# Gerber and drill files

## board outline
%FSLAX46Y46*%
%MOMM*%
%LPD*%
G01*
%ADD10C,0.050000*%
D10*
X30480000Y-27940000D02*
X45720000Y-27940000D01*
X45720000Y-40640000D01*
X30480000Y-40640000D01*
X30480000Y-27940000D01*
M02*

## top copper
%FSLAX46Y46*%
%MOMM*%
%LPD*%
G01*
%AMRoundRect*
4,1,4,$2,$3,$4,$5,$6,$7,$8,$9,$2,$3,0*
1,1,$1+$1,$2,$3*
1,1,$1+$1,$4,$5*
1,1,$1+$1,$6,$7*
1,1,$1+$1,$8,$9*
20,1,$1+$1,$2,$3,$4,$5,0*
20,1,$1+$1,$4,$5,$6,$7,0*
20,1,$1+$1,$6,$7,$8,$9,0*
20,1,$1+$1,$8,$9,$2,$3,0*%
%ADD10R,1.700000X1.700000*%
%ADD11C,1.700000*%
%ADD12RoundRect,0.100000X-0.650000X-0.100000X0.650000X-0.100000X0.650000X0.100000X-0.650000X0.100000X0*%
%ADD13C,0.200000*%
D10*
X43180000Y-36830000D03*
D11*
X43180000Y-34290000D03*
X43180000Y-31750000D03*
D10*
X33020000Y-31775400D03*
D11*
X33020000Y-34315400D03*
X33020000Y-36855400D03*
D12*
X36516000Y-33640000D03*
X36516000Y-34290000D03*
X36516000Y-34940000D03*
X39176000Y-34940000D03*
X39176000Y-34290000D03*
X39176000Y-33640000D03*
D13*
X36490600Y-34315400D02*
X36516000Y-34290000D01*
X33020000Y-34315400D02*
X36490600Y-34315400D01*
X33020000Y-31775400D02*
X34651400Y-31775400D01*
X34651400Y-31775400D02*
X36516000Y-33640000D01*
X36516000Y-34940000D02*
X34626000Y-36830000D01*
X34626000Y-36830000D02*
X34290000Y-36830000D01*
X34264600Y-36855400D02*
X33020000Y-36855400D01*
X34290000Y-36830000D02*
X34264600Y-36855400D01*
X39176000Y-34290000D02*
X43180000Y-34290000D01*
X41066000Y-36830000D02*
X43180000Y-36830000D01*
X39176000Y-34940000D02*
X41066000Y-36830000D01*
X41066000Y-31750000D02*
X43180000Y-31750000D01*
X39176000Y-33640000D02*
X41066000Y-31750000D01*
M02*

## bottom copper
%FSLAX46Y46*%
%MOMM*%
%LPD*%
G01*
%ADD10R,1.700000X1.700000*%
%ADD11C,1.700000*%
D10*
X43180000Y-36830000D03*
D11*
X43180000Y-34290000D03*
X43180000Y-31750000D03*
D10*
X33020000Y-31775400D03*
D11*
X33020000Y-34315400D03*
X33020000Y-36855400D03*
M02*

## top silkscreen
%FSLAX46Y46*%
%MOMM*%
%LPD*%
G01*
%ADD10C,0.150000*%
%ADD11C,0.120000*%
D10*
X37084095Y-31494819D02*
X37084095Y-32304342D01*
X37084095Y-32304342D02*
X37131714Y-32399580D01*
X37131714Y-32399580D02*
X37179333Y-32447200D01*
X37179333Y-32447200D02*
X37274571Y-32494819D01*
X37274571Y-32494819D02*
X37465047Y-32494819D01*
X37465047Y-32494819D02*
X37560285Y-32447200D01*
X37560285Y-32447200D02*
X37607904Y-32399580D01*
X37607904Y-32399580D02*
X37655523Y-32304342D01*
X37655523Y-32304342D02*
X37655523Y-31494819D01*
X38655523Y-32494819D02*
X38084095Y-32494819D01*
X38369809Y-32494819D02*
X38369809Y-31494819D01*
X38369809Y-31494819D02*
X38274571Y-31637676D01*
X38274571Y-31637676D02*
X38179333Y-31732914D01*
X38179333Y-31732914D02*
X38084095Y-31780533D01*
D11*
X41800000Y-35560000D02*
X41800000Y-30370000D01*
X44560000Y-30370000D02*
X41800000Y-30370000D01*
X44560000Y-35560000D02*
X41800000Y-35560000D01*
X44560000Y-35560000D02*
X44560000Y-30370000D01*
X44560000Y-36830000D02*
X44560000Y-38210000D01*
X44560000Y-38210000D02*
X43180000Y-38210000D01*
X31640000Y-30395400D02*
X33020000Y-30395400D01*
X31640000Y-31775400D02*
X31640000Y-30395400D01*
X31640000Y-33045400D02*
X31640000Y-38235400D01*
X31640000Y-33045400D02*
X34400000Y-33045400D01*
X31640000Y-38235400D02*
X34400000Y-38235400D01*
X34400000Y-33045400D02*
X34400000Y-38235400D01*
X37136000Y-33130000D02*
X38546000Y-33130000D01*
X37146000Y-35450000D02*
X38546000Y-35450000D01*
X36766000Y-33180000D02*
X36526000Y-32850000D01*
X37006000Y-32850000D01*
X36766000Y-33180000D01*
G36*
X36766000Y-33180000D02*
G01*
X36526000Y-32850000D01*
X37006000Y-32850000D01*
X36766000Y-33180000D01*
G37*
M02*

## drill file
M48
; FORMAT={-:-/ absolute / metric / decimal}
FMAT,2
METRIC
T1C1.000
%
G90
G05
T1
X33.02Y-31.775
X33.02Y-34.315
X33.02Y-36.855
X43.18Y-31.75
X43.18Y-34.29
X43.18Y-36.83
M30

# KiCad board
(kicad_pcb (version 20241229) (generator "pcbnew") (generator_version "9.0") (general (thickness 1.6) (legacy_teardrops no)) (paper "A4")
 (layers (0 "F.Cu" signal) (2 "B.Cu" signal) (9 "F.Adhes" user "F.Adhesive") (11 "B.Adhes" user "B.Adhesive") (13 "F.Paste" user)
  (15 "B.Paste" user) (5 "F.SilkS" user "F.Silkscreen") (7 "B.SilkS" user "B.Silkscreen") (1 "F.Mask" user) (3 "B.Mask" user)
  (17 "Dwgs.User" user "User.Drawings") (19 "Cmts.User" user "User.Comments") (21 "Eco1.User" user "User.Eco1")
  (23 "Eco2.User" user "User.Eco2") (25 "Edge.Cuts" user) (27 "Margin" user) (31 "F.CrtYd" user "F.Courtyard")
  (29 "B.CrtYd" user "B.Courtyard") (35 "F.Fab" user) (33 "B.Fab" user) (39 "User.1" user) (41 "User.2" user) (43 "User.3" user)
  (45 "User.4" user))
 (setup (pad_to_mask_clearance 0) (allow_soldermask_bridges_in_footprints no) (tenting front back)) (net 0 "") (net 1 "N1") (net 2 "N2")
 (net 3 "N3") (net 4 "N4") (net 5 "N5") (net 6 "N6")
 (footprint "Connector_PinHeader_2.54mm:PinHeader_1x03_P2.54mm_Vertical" (layer "F.Cu") (at 43.18 36.83 180)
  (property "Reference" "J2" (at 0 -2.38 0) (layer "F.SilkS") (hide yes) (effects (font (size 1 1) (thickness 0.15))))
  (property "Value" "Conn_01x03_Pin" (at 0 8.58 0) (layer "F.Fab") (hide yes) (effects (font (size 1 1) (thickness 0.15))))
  (fp_line (start 1.38 1.27) (end 1.38 6.46) (stroke (width 0.12) (type solid)) (layer "F.SilkS"))
  (fp_line (start -1.38 6.46) (end 1.38 6.46) (stroke (width 0.12) (type solid)) (layer "F.SilkS"))
  (fp_line (start -1.38 1.27) (end 1.38 1.27) (stroke (width 0.12) (type solid)) (layer "F.SilkS"))
  (fp_line (start -1.38 1.27) (end -1.38 6.46) (stroke (width 0.12) (type solid)) (layer "F.SilkS"))
  (fp_line (start -1.38 0) (end -1.38 -1.38) (stroke (width 0.12) (type solid)) (layer "F.SilkS"))
  (fp_line (start -1.38 -1.38) (end 0 -1.38) (stroke (width 0.12) (type solid)) (layer "F.SilkS"))
  (pad "1" thru_hole rect (at 0 0 180) (size 1.7 1.7) (drill 1) (layers "*.Cu" "*.Mask") (remove_unused_layers no) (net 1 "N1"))
  (pad "2" thru_hole circle (at 0 2.54 180) (size 1.7 1.7) (drill 1) (layers "*.Cu" "*.Mask") (remove_unused_layers no) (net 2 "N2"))
  (pad "3" thru_hole circle (at 0 5.08 180) (size 1.7 1.7) (drill 1) (layers "*.Cu" "*.Mask") (remove_unused_layers no) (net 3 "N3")))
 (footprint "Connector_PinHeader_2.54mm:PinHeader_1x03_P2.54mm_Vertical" (layer "F.Cu") (at 33.02 31.7754)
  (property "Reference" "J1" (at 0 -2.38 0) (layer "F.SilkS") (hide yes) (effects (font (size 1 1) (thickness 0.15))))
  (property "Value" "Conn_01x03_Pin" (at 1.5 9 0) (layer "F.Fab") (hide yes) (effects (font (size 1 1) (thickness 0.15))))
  (fp_line (start -1.38 -1.38) (end 0 -1.38) (stroke (width 0.12) (type solid)) (layer "F.SilkS"))
  (fp_line (start -1.38 0) (end -1.38 -1.38) (stroke (width 0.12) (type solid)) (layer "F.SilkS"))
  (fp_line (start -1.38 1.27) (end -1.38 6.46) (stroke (width 0.12) (type solid)) (layer "F.SilkS"))
  (fp_line (start -1.38 1.27) (end 1.38 1.27) (stroke (width 0.12) (type solid)) (layer "F.SilkS"))
  (fp_line (start -1.38 6.46) (end 1.38 6.46) (stroke (width 0.12) (type solid)) (layer "F.SilkS"))
  (fp_line (start 1.38 1.27) (end 1.38 6.46) (stroke (width 0.12) (type solid)) (layer "F.SilkS"))
  (pad "1" thru_hole rect (at 0 0) (size 1.7 1.7) (drill 1) (layers "*.Cu" "*.Mask") (remove_unused_layers no) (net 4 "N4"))
  (pad "2" thru_hole circle (at 0 2.54) (size 1.7 1.7) (drill 1) (layers "*.Cu" "*.Mask") (remove_unused_layers no) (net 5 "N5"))
  (pad "3" thru_hole circle (at 0 5.08) (size 1.7 1.7) (drill 1) (layers "*.Cu" "*.Mask") (remove_unused_layers no) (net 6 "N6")))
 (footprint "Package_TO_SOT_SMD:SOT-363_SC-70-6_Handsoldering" (layer "F.Cu") (at 37.846 34.29)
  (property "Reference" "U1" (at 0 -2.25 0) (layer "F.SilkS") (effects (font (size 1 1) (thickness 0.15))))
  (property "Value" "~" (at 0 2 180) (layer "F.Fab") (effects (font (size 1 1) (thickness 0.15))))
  (fp_line (start -0.71 -1.16) (end 0.7 -1.16) (stroke (width 0.12) (type solid)) (layer "F.SilkS"))
  (fp_line (start -0.7 1.16) (end 0.7 1.16) (stroke (width 0.12) (type solid)) (layer "F.SilkS"))
  (fp_poly
   (pts (xy -1.08 -1.11) (xy -1.32 -1.44) (xy -0.84 -1.44) (xy -1.08 -1.11)) (stroke (width 0.12) (type solid)) (fill yes) (layer "F.SilkS"))
  (pad "1" smd roundrect (at -1.33 -0.65) (size 1.5 0.4) (layers "F.Cu" "F.Mask" "F.Paste") (roundrect_rratio 0.25) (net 4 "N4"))
  (pad "2" smd roundrect (at -1.33 0) (size 1.5 0.4) (layers "F.Cu" "F.Mask" "F.Paste") (roundrect_rratio 0.25) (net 5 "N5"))
  (pad "3" smd roundrect (at -1.33 0.65) (size 1.5 0.4) (layers "F.Cu" "F.Mask" "F.Paste") (roundrect_rratio 0.25) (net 6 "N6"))
  (pad "4" smd roundrect (at 1.33 0.65) (size 1.5 0.4) (layers "F.Cu" "F.Mask" "F.Paste") (roundrect_rratio 0.25) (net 1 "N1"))
  (pad "5" smd roundrect (at 1.33 0) (size 1.5 0.4) (layers "F.Cu" "F.Mask" "F.Paste") (roundrect_rratio 0.25) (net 2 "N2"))
  (pad "6" smd roundrect (at 1.33 -0.65) (size 1.5 0.4) (layers "F.Cu" "F.Mask" "F.Paste") (roundrect_rratio 0.25) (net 3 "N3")))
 (gr_rect (start 30.48 27.94) (end 45.72 40.64) (stroke (width 0.05) (type default)) (fill no) (layer "Edge.Cuts"))
 (segment (start 36.4906 34.3154) (end 36.516 34.29) (width 0.2) (layer "F.Cu") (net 5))
 (segment (start 33.02 34.3154) (end 36.4906 34.3154) (width 0.2) (layer "F.Cu") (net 5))
 (segment (start 33.02 31.7754) (end 34.6514 31.7754) (width 0.2) (layer "F.Cu") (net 4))
 (segment (start 34.6514 31.7754) (end 36.516 33.64) (width 0.2) (layer "F.Cu") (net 4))
 (segment (start 36.516 34.94) (end 34.626 36.83) (width 0.2) (layer "F.Cu") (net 6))
 (segment (start 34.626 36.83) (end 34.29 36.83) (width 0.2) (layer "F.Cu") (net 6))
 (segment (start 34.2646 36.8554) (end 33.02 36.8554) (width 0.2) (layer "F.Cu") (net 6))
 (segment (start 34.29 36.83) (end 34.2646 36.8554) (width 0.2) (layer "F.Cu") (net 6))
 (segment (start 39.176 34.29) (end 43.18 34.29) (width 0.2) (layer "F.Cu") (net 2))
 (segment (start 41.066 36.83) (end 43.18 36.83) (width 0.2) (layer "F.Cu") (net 1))
 (segment (start 39.176 34.94) (end 41.066 36.83) (width 0.2) (layer "F.Cu") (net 1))
 (segment (start 41.066 31.75) (end 43.18 31.75) (width 0.2) (layer "F.Cu") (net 3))
 (segment (start 39.176 33.64) (end 41.066 31.75) (width 0.2) (layer "F.Cu") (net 3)))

